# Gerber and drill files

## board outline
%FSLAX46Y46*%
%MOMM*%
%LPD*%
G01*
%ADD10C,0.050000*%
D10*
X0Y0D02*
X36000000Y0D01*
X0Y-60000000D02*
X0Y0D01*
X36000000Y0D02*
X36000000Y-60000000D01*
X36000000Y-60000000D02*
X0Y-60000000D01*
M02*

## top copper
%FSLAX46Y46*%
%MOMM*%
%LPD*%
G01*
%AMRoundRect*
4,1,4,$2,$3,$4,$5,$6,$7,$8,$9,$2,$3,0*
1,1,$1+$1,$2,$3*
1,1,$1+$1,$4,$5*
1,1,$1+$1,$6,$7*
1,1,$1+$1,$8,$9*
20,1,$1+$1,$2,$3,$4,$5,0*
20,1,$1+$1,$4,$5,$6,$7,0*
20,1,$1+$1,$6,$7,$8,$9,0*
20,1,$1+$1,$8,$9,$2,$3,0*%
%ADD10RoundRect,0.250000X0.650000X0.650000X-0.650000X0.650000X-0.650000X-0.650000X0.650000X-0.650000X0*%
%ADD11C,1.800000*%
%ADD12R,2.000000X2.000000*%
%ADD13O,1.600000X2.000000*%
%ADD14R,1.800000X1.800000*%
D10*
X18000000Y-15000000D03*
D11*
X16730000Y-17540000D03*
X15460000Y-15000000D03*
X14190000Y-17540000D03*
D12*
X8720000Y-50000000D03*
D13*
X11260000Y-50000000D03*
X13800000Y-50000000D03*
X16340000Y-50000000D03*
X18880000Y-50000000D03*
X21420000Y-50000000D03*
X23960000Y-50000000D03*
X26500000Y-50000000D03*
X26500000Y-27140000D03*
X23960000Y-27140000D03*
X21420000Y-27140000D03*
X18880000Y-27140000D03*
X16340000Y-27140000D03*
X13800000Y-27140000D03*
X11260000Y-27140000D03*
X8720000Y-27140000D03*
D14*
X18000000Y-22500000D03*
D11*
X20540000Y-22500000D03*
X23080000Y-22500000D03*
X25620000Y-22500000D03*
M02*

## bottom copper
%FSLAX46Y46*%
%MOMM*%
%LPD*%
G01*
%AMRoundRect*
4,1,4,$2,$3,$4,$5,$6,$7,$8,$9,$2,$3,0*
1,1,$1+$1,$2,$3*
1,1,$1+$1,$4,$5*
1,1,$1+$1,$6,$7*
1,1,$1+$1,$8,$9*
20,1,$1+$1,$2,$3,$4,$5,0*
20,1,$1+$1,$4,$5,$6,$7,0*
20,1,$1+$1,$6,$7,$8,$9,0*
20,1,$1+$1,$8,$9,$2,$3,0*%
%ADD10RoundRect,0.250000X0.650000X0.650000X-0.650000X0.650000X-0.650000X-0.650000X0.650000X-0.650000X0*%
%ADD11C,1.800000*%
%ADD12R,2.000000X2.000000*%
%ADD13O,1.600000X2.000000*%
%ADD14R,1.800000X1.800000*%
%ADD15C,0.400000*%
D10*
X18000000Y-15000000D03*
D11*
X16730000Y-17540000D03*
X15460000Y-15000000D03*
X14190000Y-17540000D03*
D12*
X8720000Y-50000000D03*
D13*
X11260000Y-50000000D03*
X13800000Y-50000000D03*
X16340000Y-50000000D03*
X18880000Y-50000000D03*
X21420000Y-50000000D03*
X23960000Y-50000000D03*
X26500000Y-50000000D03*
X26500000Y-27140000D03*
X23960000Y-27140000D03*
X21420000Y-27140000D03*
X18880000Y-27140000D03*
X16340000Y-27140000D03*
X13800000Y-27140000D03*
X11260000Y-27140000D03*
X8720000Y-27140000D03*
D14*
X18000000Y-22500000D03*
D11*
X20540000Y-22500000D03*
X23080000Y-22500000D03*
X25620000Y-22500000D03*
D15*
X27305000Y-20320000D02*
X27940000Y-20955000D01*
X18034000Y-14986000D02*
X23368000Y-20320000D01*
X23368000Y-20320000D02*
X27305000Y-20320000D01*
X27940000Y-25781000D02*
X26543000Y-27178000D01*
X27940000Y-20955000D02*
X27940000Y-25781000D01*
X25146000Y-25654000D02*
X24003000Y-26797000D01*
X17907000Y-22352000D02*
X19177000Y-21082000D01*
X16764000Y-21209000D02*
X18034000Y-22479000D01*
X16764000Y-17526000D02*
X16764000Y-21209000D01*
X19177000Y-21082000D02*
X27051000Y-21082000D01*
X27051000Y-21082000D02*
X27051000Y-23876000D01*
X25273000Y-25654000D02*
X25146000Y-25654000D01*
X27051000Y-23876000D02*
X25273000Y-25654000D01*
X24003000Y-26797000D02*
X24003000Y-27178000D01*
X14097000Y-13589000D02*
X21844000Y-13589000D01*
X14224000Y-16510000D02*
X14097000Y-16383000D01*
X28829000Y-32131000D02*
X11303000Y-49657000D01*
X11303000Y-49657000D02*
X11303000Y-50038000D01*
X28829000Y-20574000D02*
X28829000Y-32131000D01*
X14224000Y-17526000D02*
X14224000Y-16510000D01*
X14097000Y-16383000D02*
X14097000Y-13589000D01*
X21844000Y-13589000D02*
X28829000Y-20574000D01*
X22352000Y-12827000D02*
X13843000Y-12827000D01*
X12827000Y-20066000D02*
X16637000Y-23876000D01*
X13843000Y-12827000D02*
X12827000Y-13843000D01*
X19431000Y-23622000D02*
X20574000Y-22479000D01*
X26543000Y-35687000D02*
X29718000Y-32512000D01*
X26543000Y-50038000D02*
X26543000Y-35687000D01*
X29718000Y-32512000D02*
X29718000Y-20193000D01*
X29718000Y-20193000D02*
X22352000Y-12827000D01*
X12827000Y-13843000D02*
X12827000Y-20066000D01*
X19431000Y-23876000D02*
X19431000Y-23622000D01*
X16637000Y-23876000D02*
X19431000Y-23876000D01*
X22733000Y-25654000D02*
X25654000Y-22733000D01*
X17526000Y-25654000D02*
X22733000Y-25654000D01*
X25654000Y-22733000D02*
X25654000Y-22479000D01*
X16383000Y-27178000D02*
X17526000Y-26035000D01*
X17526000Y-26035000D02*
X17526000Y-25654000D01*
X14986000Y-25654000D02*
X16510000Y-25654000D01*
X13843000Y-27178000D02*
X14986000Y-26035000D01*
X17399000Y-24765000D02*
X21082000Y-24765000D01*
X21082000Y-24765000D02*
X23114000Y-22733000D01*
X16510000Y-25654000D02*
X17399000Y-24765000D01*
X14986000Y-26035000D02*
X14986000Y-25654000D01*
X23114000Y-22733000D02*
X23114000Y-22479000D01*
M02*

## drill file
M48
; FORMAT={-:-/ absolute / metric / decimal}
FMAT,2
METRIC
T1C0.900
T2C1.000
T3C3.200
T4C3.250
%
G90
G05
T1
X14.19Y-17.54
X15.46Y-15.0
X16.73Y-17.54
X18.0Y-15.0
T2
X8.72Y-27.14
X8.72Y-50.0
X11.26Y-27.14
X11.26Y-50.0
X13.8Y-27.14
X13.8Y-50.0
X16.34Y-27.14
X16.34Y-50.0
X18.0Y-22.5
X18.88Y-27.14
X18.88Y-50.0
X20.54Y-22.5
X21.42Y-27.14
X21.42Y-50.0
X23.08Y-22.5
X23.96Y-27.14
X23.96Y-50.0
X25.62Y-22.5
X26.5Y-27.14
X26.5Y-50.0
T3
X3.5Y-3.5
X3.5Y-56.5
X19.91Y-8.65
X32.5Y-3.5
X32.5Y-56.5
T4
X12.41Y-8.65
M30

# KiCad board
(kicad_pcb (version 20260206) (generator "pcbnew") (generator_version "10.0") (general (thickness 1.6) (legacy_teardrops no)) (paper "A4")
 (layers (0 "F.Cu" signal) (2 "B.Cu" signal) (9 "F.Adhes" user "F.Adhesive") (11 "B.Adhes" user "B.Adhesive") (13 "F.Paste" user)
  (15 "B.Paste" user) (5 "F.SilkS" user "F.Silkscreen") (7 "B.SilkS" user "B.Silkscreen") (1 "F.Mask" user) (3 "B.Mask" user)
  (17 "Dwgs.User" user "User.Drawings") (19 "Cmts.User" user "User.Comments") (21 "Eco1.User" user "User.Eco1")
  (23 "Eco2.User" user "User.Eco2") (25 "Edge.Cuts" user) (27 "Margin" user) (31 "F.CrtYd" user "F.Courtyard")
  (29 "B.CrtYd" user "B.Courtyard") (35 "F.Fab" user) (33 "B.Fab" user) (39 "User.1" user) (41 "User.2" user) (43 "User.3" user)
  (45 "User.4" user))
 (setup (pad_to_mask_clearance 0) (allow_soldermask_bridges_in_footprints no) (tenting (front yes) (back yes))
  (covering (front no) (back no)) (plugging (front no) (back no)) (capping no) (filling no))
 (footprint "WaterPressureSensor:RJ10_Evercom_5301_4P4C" (layer "F.Cu") (at 18 15 180)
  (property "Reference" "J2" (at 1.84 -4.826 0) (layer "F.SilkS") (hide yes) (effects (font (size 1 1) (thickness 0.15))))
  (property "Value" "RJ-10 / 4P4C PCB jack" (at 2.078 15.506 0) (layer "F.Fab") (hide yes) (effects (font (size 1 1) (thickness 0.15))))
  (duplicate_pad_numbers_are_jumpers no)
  (pad "" np_thru_hole circle (at -1.91 6.35 180) (size 3.25 3.25) (drill 3.2) (layers "*.Mask"))
  (pad "" np_thru_hole circle (at 5.59 6.35 180) (size 3.25 3.25) (drill 3.25) (layers "*.Mask"))
  (pad "1" thru_hole roundrect (at 0 0 180) (size 1.8 1.8) (drill 0.9) (layers "*.Cu") (remove_unused_layers no)
   (roundrect_rratio 0.1388888889) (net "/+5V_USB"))
  (pad "2" thru_hole circle (at 1.27 -2.54 180) (size 1.8 1.8) (drill 0.9) (layers "*.Cu") (remove_unused_layers no) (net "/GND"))
  (pad "3" thru_hole circle (at 2.54 0 180) (size 1.8 1.8) (drill 0.9) (layers "*.Cu") (remove_unused_layers no)
   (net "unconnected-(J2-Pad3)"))
  (pad "4" thru_hole circle (at 3.81 -2.54 180) (size 1.8 1.8) (drill 0.9) (layers "*.Cu") (remove_unused_layers no) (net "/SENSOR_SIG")))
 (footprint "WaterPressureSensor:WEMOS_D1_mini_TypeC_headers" (layer "F.Cu") (at 8.72 50 90)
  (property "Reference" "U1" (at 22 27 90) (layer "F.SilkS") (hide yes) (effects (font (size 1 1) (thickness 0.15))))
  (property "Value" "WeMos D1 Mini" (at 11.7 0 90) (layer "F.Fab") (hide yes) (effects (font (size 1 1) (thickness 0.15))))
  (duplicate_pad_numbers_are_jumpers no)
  (pad "1" thru_hole rect (at 0 0 90) (size 2 2) (drill 1) (layers "*.Cu") (remove_unused_layers no) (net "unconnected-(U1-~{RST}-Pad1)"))
  (pad "2" thru_hole oval (at 0 2.54 90) (size 2 1.6) (drill 1) (layers "*.Cu") (remove_unused_layers no) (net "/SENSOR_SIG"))
  (pad "3" thru_hole oval (at 0 5.08 90) (size 2 1.6) (drill 1) (layers "*.Cu") (remove_unused_layers no) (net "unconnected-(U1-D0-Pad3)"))
  (pad "4" thru_hole oval (at 0 7.62 90) (size 2 1.6) (drill 1) (layers "*.Cu") (remove_unused_layers no)
   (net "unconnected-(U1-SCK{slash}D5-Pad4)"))
  (pad "5" thru_hole oval (at 0 10.16 90) (size 2 1.6) (drill 1) (layers "*.Cu") (remove_unused_layers no)
   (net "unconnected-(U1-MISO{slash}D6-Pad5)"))
  (pad "6" thru_hole oval (at 0 12.7 90) (size 2 1.6) (drill 1) (layers "*.Cu") (remove_unused_layers no)
   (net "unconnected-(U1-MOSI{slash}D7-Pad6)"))
  (pad "7" thru_hole oval (at 0 15.24 90) (size 2 1.6) (drill 1) (layers "*.Cu") (remove_unused_layers no)
   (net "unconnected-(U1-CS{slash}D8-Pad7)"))
  (pad "8" thru_hole oval (at 0 17.78 90) (size 2 1.6) (drill 1) (layers "*.Cu") (remove_unused_layers no) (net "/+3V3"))
  (pad "9" thru_hole oval (at 22.86 17.78 90) (size 2 1.6) (drill 1) (layers "*.Cu") (remove_unused_layers no) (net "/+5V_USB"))
  (pad "10" thru_hole oval (at 22.86 15.24 90) (size 2 1.6) (drill 1) (layers "*.Cu") (remove_unused_layers no) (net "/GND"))
  (pad "11" thru_hole oval (at 22.86 12.7 90) (size 2 1.6) (drill 1) (layers "*.Cu") (remove_unused_layers no)
   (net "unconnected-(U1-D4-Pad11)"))
  (pad "12" thru_hole oval (at 22.86 10.16 90) (size 2 1.6) (drill 1) (layers "*.Cu") (remove_unused_layers no)
   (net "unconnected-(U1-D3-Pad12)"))
  (pad "13" thru_hole oval (at 22.86 7.62 90) (size 2 1.6) (drill 1) (layers "*.Cu") (remove_unused_layers no) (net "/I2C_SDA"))
  (pad "14" thru_hole oval (at 22.86 5.08 90) (size 2 1.6) (drill 1) (layers "*.Cu") (remove_unused_layers no) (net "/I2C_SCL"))
  (pad "15" thru_hole oval (at 22.86 2.54 90) (size 2 1.6) (drill 1) (layers "*.Cu") (remove_unused_layers no)
   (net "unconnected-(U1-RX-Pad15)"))
  (pad "16" thru_hole oval (at 22.86 0 90) (size 2 1.6) (drill 1) (layers "*.Cu") (remove_unused_layers no)
   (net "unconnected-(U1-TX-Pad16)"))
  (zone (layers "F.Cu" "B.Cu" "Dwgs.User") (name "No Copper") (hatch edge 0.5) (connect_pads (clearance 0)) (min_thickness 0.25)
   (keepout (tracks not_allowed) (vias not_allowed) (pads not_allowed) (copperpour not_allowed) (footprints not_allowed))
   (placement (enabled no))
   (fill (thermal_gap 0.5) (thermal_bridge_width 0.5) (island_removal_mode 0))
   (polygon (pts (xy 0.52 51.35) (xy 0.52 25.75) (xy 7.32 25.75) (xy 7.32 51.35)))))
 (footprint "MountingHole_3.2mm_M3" (layer "F.Cu") (at 32.5 3.5)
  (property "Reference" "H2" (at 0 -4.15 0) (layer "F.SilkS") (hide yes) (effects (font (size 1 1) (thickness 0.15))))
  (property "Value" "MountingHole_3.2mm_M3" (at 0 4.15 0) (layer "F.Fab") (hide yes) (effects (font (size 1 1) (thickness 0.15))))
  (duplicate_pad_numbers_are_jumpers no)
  (pad "" np_thru_hole circle (at 0 0) (size 3.2 3.2) (drill 3.2) (layers "*.Cu" "F.Mask")))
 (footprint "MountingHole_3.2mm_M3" (layer "F.Cu") (at 32.5 56.5)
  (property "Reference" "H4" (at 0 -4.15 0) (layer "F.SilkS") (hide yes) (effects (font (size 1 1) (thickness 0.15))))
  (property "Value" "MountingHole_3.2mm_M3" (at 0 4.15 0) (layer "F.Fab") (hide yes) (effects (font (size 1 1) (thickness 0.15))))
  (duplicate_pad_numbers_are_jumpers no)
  (pad "" np_thru_hole circle (at 0 0) (size 3.2 3.2) (drill 3.2) (layers "*.Cu" "F.Mask")))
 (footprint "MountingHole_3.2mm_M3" (layer "F.Cu") (at 3.5 3.5)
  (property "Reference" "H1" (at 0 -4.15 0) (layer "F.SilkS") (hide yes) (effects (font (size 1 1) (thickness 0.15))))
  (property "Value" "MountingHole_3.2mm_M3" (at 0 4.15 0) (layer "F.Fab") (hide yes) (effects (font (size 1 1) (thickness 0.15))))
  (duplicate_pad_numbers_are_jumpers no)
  (pad "" np_thru_hole circle (at 0 0) (size 3.2 3.2) (drill 3.2) (layers "*.Cu" "F.Mask")))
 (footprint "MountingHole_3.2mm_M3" (layer "F.Cu") (at 3.5 56.5)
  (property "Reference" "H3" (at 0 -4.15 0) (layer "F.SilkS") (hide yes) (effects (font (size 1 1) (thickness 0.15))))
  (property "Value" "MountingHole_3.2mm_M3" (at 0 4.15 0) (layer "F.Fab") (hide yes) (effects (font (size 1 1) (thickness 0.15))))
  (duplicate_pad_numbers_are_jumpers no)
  (pad "" np_thru_hole circle (at 0 0) (size 3.2 3.2) (drill 3.2) (layers "*.Cu" "F.Mask")))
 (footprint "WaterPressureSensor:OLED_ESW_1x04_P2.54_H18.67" (layer "F.Cu") (at 18 22.5 90)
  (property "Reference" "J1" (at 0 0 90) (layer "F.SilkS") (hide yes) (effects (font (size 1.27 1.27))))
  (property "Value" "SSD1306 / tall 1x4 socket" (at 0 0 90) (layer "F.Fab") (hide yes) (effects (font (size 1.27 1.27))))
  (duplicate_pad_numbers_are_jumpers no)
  (pad "1" thru_hole rect (at 0 0 90) (size 1.8 1.8) (drill 1) (layers "*.Cu") (remove_unused_layers no) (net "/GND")
   (thermal_bridge_angle 45))
  (pad "2" thru_hole circle (at 0 2.54 90) (size 1.8 1.8) (drill 1) (layers "*.Cu") (remove_unused_layers no) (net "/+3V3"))
  (pad "3" thru_hole circle (at 0 5.08 90) (size 1.8 1.8) (drill 1) (layers "*.Cu") (remove_unused_layers no) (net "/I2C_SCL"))
  (pad "4" thru_hole circle (at 0 7.62 90) (size 1.8 1.8) (drill 1) (layers "*.Cu") (remove_unused_layers no) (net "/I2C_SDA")))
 (gr_line (start 0 0) (end 36 0) (stroke (width 0.05) (type default)) (layer "Edge.Cuts"))
 (gr_line (start 0 60) (end 0 0) (stroke (width 0.05) (type default)) (layer "Edge.Cuts"))
 (gr_line (start 36 0) (end 36 60) (stroke (width 0.05) (type default)) (layer "Edge.Cuts"))
 (gr_line (start 36 60) (end 0 60) (stroke (width 0.05) (type default)) (layer "Edge.Cuts"))
 (segment (start 27.305 20.32) (end 27.94 20.955) (width 0.4) (layer "B.Cu") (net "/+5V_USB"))
 (segment (start 18.034 14.986) (end 23.368 20.32) (width 0.4) (layer "B.Cu") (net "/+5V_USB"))
 (segment (start 23.368 20.32) (end 27.305 20.32) (width 0.4) (layer "B.Cu") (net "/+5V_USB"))
 (segment (start 27.94 25.781) (end 26.543 27.178) (width 0.4) (layer "B.Cu") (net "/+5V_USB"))
 (segment (start 27.94 20.955) (end 27.94 25.781) (width 0.4) (layer "B.Cu") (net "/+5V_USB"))
 (segment (start 25.146 25.654) (end 24.003 26.797) (width 0.4) (layer "B.Cu") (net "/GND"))
 (segment (start 17.907 22.352) (end 19.177 21.082) (width 0.4) (layer "B.Cu") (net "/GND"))
 (segment (start 16.764 21.209) (end 18.034 22.479) (width 0.4) (layer "B.Cu") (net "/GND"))
 (segment (start 16.764 17.526) (end 16.764 21.209) (width 0.4) (layer "B.Cu") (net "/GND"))
 (segment (start 19.177 21.082) (end 27.051 21.082) (width 0.4) (layer "B.Cu") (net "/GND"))
 (segment (start 27.051 21.082) (end 27.051 23.876) (width 0.4) (layer "B.Cu") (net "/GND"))
 (segment (start 25.273 25.654) (end 25.146 25.654) (width 0.4) (layer "B.Cu") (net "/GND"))
 (segment (start 27.051 23.876) (end 25.273 25.654) (width 0.4) (layer "B.Cu") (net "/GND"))
 (segment (start 24.003 26.797) (end 24.003 27.178) (width 0.4) (layer "B.Cu") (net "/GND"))
 (segment (start 14.097 13.589) (end 21.844 13.589) (width 0.4) (layer "B.Cu") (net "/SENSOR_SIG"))
 (segment (start 14.224 16.51) (end 14.097 16.383) (width 0.4) (layer "B.Cu") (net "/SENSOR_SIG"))
 (segment (start 28.829 32.131) (end 11.303 49.657) (width 0.4) (layer "B.Cu") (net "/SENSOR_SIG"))
 (segment (start 11.303 49.657) (end 11.303 50.038) (width 0.4) (layer "B.Cu") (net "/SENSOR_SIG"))
 (segment (start 28.829 20.574) (end 28.829 32.131) (width 0.4) (layer "B.Cu") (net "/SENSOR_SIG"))
 (segment (start 14.224 17.526) (end 14.224 16.51) (width 0.4) (layer "B.Cu") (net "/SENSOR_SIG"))
 (segment (start 14.097 16.383) (end 14.097 13.589) (width 0.4) (layer "B.Cu") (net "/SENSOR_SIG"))
 (segment (start 21.844 13.589) (end 28.829 20.574) (width 0.4) (layer "B.Cu") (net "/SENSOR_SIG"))
 (segment (start 22.352 12.827) (end 13.843 12.827) (width 0.4) (layer "B.Cu") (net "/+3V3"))
 (segment (start 12.827 20.066) (end 16.637 23.876) (width 0.4) (layer "B.Cu") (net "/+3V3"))
 (segment (start 13.843 12.827) (end 12.827 13.843) (width 0.4) (layer "B.Cu") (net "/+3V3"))
 (segment (start 19.431 23.622) (end 20.574 22.479) (width 0.4) (layer "B.Cu") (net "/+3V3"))
 (segment (start 26.543 35.687) (end 29.718 32.512) (width 0.4) (layer "B.Cu") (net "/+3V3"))
 (segment (start 26.543 50.038) (end 26.543 35.687) (width 0.4) (layer "B.Cu") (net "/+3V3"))
 (segment (start 29.718 32.512) (end 29.718 20.193) (width 0.4) (layer "B.Cu") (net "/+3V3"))
 (segment (start 29.718 20.193) (end 22.352 12.827) (width 0.4) (layer "B.Cu") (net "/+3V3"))
 (segment (start 12.827 13.843) (end 12.827 20.066) (width 0.4) (layer "B.Cu") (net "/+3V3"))
 (segment (start 19.431 23.876) (end 19.431 23.622) (width 0.4) (layer "B.Cu") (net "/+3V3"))
 (segment (start 16.637 23.876) (end 19.431 23.876) (width 0.4) (layer "B.Cu") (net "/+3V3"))
 (segment (start 22.733 25.654) (end 25.654 22.733) (width 0.4) (layer "B.Cu") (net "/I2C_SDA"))
 (segment (start 17.526 25.654) (end 22.733 25.654) (width 0.4) (layer "B.Cu") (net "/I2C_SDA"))
 (segment (start 25.654 22.733) (end 25.654 22.479) (width 0.4) (layer "B.Cu") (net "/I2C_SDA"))
 (segment (start 16.383 27.178) (end 17.526 26.035) (width 0.4) (layer "B.Cu") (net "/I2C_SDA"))
 (segment (start 17.526 26.035) (end 17.526 25.654) (width 0.4) (layer "B.Cu") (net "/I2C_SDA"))
 (segment (start 14.986 25.654) (end 16.51 25.654) (width 0.4) (layer "B.Cu") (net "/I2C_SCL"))
 (segment (start 13.843 27.178) (end 14.986 26.035) (width 0.4) (layer "B.Cu") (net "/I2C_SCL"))
 (segment (start 17.399 24.765) (end 21.082 24.765) (width 0.4) (layer "B.Cu") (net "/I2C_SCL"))
 (segment (start 21.082 24.765) (end 23.114 22.733) (width 0.4) (layer "B.Cu") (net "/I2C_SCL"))
 (segment (start 16.51 25.654) (end 17.399 24.765) (width 0.4) (layer "B.Cu") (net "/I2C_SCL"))
 (segment (start 14.986 26.035) (end 14.986 25.654) (width 0.4) (layer "B.Cu") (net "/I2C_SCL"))
 (segment (start 23.114 22.733) (end 23.114 22.479) (width 0.4) (layer "B.Cu") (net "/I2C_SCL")))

